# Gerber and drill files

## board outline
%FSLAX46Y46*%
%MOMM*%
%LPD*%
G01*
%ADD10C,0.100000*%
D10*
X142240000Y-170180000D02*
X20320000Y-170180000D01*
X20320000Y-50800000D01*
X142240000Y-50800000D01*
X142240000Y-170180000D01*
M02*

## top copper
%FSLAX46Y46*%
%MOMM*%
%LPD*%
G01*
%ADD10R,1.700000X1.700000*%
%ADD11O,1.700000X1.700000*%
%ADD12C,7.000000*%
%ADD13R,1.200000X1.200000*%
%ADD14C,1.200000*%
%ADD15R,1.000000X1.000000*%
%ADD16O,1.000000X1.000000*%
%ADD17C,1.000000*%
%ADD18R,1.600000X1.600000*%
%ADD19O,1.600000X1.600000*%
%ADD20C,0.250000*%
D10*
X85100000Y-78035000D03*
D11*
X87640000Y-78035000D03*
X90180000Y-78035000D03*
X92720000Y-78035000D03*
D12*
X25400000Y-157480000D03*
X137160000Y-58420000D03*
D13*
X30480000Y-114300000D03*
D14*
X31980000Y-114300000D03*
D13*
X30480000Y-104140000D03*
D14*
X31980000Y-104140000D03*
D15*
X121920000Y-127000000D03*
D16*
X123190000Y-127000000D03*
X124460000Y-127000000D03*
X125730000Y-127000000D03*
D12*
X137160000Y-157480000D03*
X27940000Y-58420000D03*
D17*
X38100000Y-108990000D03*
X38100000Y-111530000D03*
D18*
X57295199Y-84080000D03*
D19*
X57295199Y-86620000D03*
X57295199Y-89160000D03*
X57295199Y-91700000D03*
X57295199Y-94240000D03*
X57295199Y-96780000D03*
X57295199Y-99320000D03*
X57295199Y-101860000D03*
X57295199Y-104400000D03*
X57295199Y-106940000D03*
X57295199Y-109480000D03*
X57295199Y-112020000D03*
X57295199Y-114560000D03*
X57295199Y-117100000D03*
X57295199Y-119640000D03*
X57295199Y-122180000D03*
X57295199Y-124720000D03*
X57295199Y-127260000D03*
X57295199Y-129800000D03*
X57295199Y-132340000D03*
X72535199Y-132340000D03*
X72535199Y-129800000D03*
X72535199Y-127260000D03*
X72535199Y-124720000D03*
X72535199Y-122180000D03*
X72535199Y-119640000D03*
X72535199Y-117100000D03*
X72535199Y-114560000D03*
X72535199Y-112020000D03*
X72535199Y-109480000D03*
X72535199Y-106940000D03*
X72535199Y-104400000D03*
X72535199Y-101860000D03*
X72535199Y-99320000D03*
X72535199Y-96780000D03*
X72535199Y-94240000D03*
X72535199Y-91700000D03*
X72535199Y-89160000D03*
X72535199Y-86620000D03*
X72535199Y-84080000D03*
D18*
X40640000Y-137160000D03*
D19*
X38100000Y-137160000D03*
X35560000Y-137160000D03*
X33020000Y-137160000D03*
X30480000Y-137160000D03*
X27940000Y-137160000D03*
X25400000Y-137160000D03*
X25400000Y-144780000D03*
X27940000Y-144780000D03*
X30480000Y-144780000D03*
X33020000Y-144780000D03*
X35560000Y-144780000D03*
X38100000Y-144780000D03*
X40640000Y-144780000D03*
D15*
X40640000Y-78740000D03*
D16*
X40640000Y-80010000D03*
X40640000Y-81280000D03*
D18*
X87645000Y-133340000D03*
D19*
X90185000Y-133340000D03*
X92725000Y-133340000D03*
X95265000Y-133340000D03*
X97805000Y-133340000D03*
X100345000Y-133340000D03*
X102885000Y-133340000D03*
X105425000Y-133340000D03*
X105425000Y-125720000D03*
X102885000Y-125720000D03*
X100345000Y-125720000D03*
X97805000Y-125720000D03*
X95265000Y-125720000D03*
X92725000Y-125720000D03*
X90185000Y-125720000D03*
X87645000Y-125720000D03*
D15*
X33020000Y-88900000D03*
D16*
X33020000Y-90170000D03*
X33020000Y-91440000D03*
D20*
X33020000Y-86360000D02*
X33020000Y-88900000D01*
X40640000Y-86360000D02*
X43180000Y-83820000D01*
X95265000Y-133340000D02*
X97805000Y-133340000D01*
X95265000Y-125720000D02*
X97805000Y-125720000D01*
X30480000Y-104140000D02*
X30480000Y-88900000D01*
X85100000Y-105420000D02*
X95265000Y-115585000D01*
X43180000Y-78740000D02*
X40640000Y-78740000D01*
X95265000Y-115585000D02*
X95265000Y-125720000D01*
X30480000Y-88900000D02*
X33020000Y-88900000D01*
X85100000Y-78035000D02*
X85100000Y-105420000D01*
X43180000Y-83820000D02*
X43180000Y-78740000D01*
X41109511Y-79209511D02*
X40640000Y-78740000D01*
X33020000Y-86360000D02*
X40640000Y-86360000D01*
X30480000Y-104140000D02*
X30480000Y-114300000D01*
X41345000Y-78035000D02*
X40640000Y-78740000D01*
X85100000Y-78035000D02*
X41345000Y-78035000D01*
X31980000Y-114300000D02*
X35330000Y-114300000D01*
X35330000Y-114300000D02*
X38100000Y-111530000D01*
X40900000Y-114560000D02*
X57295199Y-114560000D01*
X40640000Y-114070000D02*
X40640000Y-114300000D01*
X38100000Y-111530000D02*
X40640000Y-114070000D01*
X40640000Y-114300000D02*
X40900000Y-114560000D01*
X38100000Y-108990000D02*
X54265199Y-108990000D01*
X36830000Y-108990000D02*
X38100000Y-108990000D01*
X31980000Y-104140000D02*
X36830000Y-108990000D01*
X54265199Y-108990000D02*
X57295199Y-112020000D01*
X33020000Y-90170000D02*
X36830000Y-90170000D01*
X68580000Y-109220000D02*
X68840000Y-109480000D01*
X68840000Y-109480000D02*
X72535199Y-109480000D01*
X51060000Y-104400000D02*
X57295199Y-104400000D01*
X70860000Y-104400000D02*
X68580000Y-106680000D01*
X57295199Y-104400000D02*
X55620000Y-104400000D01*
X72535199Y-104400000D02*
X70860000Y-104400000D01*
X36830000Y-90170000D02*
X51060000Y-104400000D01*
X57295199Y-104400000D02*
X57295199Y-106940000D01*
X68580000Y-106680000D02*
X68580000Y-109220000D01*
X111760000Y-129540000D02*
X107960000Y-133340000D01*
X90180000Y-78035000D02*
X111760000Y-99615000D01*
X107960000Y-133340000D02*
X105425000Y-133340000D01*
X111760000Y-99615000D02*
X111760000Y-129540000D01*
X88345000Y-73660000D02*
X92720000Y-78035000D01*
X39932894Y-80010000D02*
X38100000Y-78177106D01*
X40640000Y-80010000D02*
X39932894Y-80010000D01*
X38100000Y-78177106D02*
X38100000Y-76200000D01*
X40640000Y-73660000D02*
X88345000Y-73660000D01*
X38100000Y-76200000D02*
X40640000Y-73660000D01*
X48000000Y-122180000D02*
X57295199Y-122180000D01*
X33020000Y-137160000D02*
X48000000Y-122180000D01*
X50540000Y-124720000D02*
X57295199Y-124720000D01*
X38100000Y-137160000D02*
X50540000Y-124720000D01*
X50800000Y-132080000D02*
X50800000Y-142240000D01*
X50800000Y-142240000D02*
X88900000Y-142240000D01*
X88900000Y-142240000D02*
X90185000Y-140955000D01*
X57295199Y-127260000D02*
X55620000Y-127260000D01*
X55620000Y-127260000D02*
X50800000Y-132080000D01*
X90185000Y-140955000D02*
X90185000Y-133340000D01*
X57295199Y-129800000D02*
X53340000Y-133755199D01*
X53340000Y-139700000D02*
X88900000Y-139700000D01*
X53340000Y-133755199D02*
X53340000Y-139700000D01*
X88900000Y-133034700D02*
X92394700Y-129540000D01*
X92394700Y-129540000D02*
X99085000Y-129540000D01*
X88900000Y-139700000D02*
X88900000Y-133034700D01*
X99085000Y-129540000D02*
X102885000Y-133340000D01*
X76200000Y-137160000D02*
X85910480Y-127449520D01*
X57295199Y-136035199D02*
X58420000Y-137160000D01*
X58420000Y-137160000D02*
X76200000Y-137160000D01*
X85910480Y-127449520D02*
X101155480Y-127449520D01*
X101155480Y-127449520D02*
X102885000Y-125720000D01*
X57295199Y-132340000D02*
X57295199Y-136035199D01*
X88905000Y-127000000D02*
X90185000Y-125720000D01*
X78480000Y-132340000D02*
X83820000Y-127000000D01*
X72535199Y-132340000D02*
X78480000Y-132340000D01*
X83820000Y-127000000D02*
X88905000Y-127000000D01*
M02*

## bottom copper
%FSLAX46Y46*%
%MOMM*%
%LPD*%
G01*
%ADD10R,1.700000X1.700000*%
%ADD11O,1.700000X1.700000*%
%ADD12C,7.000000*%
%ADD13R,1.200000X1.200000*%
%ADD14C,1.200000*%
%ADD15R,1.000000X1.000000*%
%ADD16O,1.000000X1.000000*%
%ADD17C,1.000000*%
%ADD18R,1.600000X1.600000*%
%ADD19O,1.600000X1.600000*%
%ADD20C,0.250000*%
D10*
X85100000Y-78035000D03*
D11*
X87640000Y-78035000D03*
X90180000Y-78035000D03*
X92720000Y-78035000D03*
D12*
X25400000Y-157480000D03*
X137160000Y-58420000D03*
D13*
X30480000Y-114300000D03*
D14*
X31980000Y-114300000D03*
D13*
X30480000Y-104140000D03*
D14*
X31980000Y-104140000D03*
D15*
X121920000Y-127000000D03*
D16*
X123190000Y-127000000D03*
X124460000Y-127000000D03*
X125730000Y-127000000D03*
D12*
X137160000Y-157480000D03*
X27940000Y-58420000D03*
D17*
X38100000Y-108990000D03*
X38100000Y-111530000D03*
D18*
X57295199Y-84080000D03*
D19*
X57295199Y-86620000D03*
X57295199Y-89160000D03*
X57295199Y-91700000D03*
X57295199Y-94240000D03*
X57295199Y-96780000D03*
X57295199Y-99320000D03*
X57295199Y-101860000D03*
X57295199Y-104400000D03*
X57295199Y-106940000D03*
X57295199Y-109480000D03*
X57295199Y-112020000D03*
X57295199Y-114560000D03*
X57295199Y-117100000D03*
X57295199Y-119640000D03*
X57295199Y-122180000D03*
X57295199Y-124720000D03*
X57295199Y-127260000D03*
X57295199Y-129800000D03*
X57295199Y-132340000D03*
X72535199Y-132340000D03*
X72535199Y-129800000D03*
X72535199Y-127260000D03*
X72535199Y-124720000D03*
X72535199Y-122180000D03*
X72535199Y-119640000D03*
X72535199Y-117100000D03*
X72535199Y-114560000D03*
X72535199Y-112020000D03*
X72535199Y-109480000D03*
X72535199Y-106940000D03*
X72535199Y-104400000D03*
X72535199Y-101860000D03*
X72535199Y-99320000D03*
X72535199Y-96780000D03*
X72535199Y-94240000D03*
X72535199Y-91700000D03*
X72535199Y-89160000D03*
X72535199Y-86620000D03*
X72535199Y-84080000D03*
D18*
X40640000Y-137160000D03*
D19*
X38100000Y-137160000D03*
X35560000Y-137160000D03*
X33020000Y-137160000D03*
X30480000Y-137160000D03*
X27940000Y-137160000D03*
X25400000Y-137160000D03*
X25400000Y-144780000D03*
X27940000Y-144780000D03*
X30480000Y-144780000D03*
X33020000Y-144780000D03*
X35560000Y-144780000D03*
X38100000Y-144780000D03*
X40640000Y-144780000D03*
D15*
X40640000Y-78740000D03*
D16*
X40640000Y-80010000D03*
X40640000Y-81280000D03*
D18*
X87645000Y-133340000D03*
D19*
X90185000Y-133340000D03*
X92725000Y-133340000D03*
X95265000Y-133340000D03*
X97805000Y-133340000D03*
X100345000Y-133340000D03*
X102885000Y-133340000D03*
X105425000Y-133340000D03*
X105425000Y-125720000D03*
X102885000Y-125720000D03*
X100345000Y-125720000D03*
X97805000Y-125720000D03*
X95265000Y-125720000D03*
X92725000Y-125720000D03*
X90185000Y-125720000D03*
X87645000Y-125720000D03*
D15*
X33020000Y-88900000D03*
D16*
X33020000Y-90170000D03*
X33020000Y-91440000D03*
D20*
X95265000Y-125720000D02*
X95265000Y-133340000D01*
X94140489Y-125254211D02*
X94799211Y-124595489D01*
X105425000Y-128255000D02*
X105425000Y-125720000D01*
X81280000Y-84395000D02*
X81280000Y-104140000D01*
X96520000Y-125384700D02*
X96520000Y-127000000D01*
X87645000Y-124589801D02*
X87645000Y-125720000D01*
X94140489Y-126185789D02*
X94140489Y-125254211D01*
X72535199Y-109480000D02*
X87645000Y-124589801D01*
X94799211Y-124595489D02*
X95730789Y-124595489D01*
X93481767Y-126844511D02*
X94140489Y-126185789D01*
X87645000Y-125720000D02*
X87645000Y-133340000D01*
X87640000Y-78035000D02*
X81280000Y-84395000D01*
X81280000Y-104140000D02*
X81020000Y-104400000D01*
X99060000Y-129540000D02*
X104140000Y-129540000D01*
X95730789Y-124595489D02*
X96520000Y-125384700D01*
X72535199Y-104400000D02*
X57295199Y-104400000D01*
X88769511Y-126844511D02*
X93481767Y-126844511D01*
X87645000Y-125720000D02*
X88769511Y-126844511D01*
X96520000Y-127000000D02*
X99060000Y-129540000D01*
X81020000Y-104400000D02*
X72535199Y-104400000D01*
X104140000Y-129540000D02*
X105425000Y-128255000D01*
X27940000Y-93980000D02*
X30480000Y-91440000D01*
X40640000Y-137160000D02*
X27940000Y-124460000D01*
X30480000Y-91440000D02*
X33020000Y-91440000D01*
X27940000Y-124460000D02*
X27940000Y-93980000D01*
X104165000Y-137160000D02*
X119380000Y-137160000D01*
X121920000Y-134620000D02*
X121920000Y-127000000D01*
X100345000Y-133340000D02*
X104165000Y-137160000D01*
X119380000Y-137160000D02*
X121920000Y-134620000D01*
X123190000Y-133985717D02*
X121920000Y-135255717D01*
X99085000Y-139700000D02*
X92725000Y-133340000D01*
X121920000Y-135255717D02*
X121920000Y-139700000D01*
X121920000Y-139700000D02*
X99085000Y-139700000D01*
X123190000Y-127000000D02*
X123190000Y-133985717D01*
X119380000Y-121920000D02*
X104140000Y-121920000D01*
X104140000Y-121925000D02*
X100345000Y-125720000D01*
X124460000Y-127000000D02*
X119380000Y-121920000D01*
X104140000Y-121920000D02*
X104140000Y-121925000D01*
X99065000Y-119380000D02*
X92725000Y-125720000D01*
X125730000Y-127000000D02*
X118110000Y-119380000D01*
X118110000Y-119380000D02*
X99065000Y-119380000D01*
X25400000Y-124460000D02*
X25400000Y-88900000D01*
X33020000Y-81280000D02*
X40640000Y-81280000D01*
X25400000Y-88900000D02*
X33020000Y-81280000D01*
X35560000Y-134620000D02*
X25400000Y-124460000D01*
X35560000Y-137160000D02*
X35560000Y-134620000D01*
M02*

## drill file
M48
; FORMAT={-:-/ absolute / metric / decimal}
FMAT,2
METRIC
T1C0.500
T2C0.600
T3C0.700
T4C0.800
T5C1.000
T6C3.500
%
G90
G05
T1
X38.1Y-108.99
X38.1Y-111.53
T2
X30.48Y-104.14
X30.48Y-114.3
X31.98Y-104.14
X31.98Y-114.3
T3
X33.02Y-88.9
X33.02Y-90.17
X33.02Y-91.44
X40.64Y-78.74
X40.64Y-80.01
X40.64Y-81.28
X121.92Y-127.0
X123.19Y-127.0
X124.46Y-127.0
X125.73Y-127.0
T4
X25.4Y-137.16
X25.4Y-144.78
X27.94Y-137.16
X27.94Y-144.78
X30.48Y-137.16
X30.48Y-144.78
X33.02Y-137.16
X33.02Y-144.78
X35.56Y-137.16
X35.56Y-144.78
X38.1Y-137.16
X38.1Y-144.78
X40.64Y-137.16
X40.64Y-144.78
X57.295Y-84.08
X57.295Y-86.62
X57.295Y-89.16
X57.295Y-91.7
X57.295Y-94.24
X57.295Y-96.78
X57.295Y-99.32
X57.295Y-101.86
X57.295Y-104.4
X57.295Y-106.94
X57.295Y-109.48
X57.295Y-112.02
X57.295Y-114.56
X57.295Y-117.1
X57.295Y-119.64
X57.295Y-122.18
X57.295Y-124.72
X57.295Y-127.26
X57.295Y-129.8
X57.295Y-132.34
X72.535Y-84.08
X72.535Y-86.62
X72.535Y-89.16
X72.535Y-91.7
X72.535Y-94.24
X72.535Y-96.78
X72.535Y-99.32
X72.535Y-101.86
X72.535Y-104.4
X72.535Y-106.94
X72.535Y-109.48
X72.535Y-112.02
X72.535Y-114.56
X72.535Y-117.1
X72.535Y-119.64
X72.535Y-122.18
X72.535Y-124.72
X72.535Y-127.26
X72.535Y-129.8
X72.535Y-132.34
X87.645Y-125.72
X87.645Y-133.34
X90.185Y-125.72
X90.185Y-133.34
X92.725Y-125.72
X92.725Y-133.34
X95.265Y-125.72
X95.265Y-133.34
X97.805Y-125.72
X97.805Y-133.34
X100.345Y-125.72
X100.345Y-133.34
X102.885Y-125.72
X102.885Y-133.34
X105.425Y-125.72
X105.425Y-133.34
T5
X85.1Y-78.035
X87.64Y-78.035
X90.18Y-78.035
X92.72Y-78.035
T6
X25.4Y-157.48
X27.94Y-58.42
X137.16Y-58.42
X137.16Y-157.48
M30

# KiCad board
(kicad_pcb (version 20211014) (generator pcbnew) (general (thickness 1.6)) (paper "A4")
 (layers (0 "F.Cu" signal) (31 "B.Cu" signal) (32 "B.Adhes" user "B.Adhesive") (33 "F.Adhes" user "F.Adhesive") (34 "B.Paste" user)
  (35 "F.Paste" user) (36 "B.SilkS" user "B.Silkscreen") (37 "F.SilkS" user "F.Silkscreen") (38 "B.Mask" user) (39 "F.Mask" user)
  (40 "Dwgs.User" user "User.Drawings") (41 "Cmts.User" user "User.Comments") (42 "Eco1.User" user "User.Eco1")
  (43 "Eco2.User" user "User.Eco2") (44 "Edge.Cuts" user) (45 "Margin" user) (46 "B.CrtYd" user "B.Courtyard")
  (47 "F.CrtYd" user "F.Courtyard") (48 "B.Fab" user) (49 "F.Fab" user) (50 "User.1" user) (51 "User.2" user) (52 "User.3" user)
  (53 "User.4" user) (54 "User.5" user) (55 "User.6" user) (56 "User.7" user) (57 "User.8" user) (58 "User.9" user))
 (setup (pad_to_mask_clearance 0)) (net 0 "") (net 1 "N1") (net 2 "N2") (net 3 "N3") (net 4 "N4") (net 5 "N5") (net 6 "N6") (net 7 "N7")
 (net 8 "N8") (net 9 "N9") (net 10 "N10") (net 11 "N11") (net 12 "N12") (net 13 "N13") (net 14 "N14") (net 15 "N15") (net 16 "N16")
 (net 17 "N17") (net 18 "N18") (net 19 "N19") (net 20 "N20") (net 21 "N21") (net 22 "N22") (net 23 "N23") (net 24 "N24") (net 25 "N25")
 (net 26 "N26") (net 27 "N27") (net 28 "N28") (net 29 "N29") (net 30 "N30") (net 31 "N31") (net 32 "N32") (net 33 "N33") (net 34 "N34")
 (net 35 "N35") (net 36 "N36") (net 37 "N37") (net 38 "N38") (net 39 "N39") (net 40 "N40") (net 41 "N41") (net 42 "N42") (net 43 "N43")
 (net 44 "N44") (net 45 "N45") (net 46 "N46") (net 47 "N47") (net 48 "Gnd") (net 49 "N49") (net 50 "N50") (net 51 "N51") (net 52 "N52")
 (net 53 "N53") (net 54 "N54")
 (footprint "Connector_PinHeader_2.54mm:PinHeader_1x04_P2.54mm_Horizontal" (layer "F.Cu") (at 85.1 78.035 90)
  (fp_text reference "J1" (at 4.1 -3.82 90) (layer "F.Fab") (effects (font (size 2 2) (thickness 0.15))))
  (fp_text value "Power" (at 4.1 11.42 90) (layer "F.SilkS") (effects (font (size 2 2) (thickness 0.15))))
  (pad "1" thru_hole rect (at 0 0 90) (size 1.7 1.7) (drill 1) (layers *.Cu *.Mask) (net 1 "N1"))
  (pad "2" thru_hole oval (at 0 2.54 90) (size 1.7 1.7) (drill 1) (layers *.Cu *.Mask) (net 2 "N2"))
  (pad "3" thru_hole oval (at 0 5.08 90) (size 1.7 1.7) (drill 1) (layers *.Cu *.Mask) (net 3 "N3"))
  (pad "4" thru_hole oval (at 0 7.62 90) (size 1.7 1.7) (drill 1) (layers *.Cu *.Mask) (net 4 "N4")))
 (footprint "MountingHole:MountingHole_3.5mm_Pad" (layer "F.Cu") (at 25.4 157.48)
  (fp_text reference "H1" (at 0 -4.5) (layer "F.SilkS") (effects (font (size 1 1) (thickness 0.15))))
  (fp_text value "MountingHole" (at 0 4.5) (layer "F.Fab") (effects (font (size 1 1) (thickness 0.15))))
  (pad "1" thru_hole circle (at 0 0) (size 7 7) (drill 3.5) (layers *.Cu *.Mask)))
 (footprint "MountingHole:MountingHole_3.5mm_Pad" (layer "F.Cu") (at 137.16 58.42)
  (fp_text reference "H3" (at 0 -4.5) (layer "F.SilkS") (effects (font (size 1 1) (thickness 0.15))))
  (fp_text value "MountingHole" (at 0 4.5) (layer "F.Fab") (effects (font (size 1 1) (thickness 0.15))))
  (pad "1" thru_hole circle (at 0 0) (size 7 7) (drill 3.5) (layers *.Cu *.Mask)))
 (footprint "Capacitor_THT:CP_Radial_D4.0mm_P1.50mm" (layer "F.Cu") (at 30.48 114.3)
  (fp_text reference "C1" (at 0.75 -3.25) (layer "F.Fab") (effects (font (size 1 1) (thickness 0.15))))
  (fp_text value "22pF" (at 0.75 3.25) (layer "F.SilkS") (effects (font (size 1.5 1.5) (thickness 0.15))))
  (pad "1" thru_hole rect (at 0 0) (size 1.2 1.2) (drill 0.6) (layers *.Cu *.Mask) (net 1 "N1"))
  (pad "2" thru_hole circle (at 1.5 0) (size 1.2 1.2) (drill 0.6) (layers *.Cu *.Mask) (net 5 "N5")))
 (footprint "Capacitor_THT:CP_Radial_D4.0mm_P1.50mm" (layer "F.Cu") (at 30.48 104.14)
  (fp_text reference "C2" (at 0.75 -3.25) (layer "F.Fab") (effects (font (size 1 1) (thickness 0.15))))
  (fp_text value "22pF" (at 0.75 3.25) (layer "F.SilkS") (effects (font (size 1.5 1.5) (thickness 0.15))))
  (pad "1" thru_hole rect (at 0 0) (size 1.2 1.2) (drill 0.6) (layers *.Cu *.Mask) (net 1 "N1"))
  (pad "2" thru_hole circle (at 1.5 0) (size 1.2 1.2) (drill 0.6) (layers *.Cu *.Mask) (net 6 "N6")))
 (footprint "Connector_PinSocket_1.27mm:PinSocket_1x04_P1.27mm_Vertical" (layer "F.Cu") (at 121.92 127 90)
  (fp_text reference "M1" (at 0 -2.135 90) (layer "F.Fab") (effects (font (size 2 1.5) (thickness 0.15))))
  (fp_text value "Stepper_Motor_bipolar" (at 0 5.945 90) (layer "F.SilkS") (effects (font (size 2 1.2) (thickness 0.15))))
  (pad "1" thru_hole rect (at 0 0 90) (size 1 1) (drill 0.7) (layers *.Cu *.Mask) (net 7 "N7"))
  (pad "2" thru_hole oval (at 0 1.27 90) (size 1 1) (drill 0.7) (layers *.Cu *.Mask) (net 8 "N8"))
  (pad "3" thru_hole oval (at 0 2.54 90) (size 1 1) (drill 0.7) (layers *.Cu *.Mask) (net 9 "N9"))
  (pad "4" thru_hole oval (at 0 3.81 90) (size 1 1) (drill 0.7) (layers *.Cu *.Mask) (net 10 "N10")))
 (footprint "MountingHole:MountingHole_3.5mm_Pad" (layer "F.Cu") (at 137.16 157.48)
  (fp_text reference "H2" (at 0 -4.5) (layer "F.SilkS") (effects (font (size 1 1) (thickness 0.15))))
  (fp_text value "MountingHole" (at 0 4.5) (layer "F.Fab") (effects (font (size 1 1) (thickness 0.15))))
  (pad "1" thru_hole circle (at 0 0) (size 7 7) (drill 3.5) (layers *.Cu *.Mask)))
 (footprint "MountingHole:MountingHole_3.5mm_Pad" (layer "F.Cu") (at 27.94 58.42)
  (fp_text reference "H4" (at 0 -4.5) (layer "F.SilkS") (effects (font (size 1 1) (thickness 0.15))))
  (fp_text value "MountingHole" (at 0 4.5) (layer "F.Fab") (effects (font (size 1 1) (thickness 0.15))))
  (pad "1" thru_hole circle (at 0 0) (size 7 7) (drill 3.5) (layers *.Cu *.Mask)))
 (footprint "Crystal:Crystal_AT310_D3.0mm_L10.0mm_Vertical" (layer "F.Cu") (at 38.1 108.99 -90)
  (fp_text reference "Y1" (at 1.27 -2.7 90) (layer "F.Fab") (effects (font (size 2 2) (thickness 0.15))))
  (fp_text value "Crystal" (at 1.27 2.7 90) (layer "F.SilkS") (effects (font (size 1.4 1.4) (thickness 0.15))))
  (pad "1" thru_hole circle (at 0 0 270) (size 1 1) (drill 0.5) (layers *.Cu *.Mask) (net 6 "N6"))
  (pad "2" thru_hole circle (at 2.54 0 270) (size 1 1) (drill 0.5) (layers *.Cu *.Mask) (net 5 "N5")))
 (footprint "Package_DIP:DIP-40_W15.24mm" (layer "F.Cu") (at 57.295199 84.08)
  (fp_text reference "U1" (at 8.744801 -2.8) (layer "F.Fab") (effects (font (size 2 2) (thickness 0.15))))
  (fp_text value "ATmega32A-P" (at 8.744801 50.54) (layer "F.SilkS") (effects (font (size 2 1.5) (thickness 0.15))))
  (pad "1" thru_hole rect (at 0 0) (size 1.6 1.6) (drill 0.8) (layers *.Cu *.Mask) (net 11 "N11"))
  (pad "2" thru_hole oval (at 0 2.54) (size 1.6 1.6) (drill 0.8) (layers *.Cu *.Mask) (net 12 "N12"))
  (pad "3" thru_hole oval (at 0 5.08) (size 1.6 1.6) (drill 0.8) (layers *.Cu *.Mask) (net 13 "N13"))
  (pad "4" thru_hole oval (at 0 7.62) (size 1.6 1.6) (drill 0.8) (layers *.Cu *.Mask) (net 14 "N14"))
  (pad "5" thru_hole oval (at 0 10.16) (size 1.6 1.6) (drill 0.8) (layers *.Cu *.Mask) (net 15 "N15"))
  (pad "6" thru_hole oval (at 0 12.7) (size 1.6 1.6) (drill 0.8) (layers *.Cu *.Mask) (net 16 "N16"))
  (pad "7" thru_hole oval (at 0 15.24) (size 1.6 1.6) (drill 0.8) (layers *.Cu *.Mask) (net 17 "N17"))
  (pad "8" thru_hole oval (at 0 17.78) (size 1.6 1.6) (drill 0.8) (layers *.Cu *.Mask) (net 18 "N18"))
  (pad "9" thru_hole oval (at 0 20.32) (size 1.6 1.6) (drill 0.8) (layers *.Cu *.Mask) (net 2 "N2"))
  (pad "10" thru_hole oval (at 0 22.86) (size 1.6 1.6) (drill 0.8) (layers *.Cu *.Mask) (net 2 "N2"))
  (pad "11" thru_hole oval (at 0 25.4) (size 1.6 1.6) (drill 0.8) (layers *.Cu *.Mask) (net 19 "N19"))
  (pad "12" thru_hole oval (at 0 27.94) (size 1.6 1.6) (drill 0.8) (layers *.Cu *.Mask) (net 6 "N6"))
  (pad "13" thru_hole oval (at 0 30.48) (size 1.6 1.6) (drill 0.8) (layers *.Cu *.Mask) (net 5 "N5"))
  (pad "14" thru_hole oval (at 0 33.02) (size 1.6 1.6) (drill 0.8) (layers *.Cu *.Mask) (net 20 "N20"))
  (pad "15" thru_hole oval (at 0 35.56) (size 1.6 1.6) (drill 0.8) (layers *.Cu *.Mask) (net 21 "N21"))
  (pad "16" thru_hole oval (at 0 38.1) (size 1.6 1.6) (drill 0.8) (layers *.Cu *.Mask) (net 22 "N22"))
  (pad "17" thru_hole oval (at 0 40.64) (size 1.6 1.6) (drill 0.8) (layers *.Cu *.Mask) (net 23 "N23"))
  (pad "18" thru_hole oval (at 0 43.18) (size 1.6 1.6) (drill 0.8) (layers *.Cu *.Mask) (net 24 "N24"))
  (pad "19" thru_hole oval (at 0 45.72) (size 1.6 1.6) (drill 0.8) (layers *.Cu *.Mask) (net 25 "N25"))
  (pad "20" thru_hole oval (at 0 48.26) (size 1.6 1.6) (drill 0.8) (layers *.Cu *.Mask) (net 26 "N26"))
  (pad "21" thru_hole oval (at 15.24 48.26) (size 1.6 1.6) (drill 0.8) (layers *.Cu *.Mask) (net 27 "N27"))
  (pad "22" thru_hole oval (at 15.24 45.72) (size 1.6 1.6) (drill 0.8) (layers *.Cu *.Mask) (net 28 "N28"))
  (pad "23" thru_hole oval (at 15.24 43.18) (size 1.6 1.6) (drill 0.8) (layers *.Cu *.Mask) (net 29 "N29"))
  (pad "24" thru_hole oval (at 15.24 40.64) (size 1.6 1.6) (drill 0.8) (layers *.Cu *.Mask) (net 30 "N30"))
  (pad "25" thru_hole oval (at 15.24 38.1) (size 1.6 1.6) (drill 0.8) (layers *.Cu *.Mask) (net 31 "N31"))
  (pad "26" thru_hole oval (at 15.24 35.56) (size 1.6 1.6) (drill 0.8) (layers *.Cu *.Mask) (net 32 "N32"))
  (pad "27" thru_hole oval (at 15.24 33.02) (size 1.6 1.6) (drill 0.8) (layers *.Cu *.Mask) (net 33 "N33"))
  (pad "28" thru_hole oval (at 15.24 30.48) (size 1.6 1.6) (drill 0.8) (layers *.Cu *.Mask) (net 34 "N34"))
  (pad "29" thru_hole oval (at 15.24 27.94) (size 1.6 1.6) (drill 0.8) (layers *.Cu *.Mask) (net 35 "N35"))
  (pad "30" thru_hole oval (at 15.24 25.4) (size 1.6 1.6) (drill 0.8) (layers *.Cu *.Mask) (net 2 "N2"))
  (pad "31" thru_hole oval (at 15.24 22.86) (size 1.6 1.6) (drill 0.8) (layers *.Cu *.Mask) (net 19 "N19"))
  (pad "32" thru_hole oval (at 15.24 20.32) (size 1.6 1.6) (drill 0.8) (layers *.Cu *.Mask) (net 2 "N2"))
  (pad "33" thru_hole oval (at 15.24 17.78) (size 1.6 1.6) (drill 0.8) (layers *.Cu *.Mask) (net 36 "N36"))
  (pad "34" thru_hole oval (at 15.24 15.24) (size 1.6 1.6) (drill 0.8) (layers *.Cu *.Mask) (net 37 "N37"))
  (pad "35" thru_hole oval (at 15.24 12.7) (size 1.6 1.6) (drill 0.8) (layers *.Cu *.Mask) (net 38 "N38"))
  (pad "36" thru_hole oval (at 15.24 10.16) (size 1.6 1.6) (drill 0.8) (layers *.Cu *.Mask) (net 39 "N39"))
  (pad "37" thru_hole oval (at 15.24 7.62) (size 1.6 1.6) (drill 0.8) (layers *.Cu *.Mask) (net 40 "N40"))
  (pad "38" thru_hole oval (at 15.24 5.08) (size 1.6 1.6) (drill 0.8) (layers *.Cu *.Mask) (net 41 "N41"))
  (pad "39" thru_hole oval (at 15.24 2.54) (size 1.6 1.6) (drill 0.8) (layers *.Cu *.Mask) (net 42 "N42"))
  (pad "40" thru_hole oval (at 15.24 0) (size 1.6 1.6) (drill 0.8) (layers *.Cu *.Mask) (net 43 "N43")))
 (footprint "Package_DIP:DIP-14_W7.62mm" (layer "F.Cu") (at 40.64 137.16 -90)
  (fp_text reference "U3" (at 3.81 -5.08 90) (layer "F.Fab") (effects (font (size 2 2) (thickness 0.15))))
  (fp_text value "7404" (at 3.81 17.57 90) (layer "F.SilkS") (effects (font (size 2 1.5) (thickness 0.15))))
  (pad "1" thru_hole rect (at 0 0 270) (size 1.6 1.6) (drill 0.8) (layers *.Cu *.Mask) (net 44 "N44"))
  (pad "2" thru_hole oval (at 0 2.54 270) (size 1.6 1.6) (drill 0.8) (layers *.Cu *.Mask) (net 23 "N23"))
  (pad "3" thru_hole oval (at 0 5.08 270) (size 1.6 1.6) (drill 0.8) (layers *.Cu *.Mask) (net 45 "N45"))
  (pad "4" thru_hole oval (at 0 7.62 270) (size 1.6 1.6) (drill 0.8) (layers *.Cu *.Mask) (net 22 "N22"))
  (pad "5" thru_hole oval (at 0 10.16 270) (size 1.6 1.6) (drill 0.8) (layers *.Cu *.Mask) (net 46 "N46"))
  (pad "6" thru_hole oval (at 0 12.7 270) (size 1.6 1.6) (drill 0.8) (layers *.Cu *.Mask) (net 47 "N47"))
  (pad "7" thru_hole oval (at 0 15.24 270) (size 1.6 1.6) (drill 0.8) (layers *.Cu *.Mask) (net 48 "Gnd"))
  (pad "8" thru_hole oval (at 7.62 15.24 270) (size 1.6 1.6) (drill 0.8) (layers *.Cu *.Mask) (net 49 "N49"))
  (pad "9" thru_hole oval (at 7.62 12.7 270) (size 1.6 1.6) (drill 0.8) (layers *.Cu *.Mask) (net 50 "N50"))
  (pad "10" thru_hole oval (at 7.62 10.16 270) (size 1.6 1.6) (drill 0.8) (layers *.Cu *.Mask) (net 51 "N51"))
  (pad "11" thru_hole oval (at 7.62 7.62 270) (size 1.6 1.6) (drill 0.8) (layers *.Cu *.Mask) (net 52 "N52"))
  (pad "12" thru_hole oval (at 7.62 5.08 270) (size 1.6 1.6) (drill 0.8) (layers *.Cu *.Mask) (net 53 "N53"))
  (pad "13" thru_hole oval (at 7.62 2.54 270) (size 1.6 1.6) (drill 0.8) (layers *.Cu *.Mask) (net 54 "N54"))
  (pad "14" thru_hole oval (at 7.62 0 270) (size 1.6 1.6) (drill 0.8) (layers *.Cu *.Mask) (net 48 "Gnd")))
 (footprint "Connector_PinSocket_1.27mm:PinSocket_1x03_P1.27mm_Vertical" (layer "F.Cu") (at 40.64 78.74)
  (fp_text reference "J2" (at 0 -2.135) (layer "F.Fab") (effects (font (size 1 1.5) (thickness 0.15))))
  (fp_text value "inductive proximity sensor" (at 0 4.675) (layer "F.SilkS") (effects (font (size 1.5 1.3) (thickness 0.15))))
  (pad "1" thru_hole rect (at 0 0) (size 1 1) (drill 0.7) (layers *.Cu *.Mask) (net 1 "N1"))
  (pad "2" thru_hole oval (at 0 1.27) (size 1 1) (drill 0.7) (layers *.Cu *.Mask) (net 4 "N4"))
  (pad "3" thru_hole oval (at 0 2.54) (size 1 1) (drill 0.7) (layers *.Cu *.Mask) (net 45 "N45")))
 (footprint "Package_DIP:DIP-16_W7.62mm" (layer "F.Cu") (at 87.645 133.34 90)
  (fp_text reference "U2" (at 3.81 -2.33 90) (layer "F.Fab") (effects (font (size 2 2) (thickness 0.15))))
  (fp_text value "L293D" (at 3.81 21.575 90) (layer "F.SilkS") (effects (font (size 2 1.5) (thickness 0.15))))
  (pad "1" thru_hole rect (at 0 0 90) (size 1.6 1.6) (drill 0.8) (layers *.Cu *.Mask) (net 2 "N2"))
  (pad "2" thru_hole oval (at 0 2.54 90) (size 1.6 1.6) (drill 0.8) (layers *.Cu *.Mask) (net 24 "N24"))
  (pad "3" thru_hole oval (at 0 5.08 90) (size 1.6 1.6) (drill 0.8) (layers *.Cu *.Mask) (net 8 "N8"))
  (pad "4" thru_hole oval (at 0 7.62 90) (size 1.6 1.6) (drill 0.8) (layers *.Cu *.Mask) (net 1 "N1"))
  (pad "5" thru_hole oval (at 0 10.16 90) (size 1.6 1.6) (drill 0.8) (layers *.Cu *.Mask) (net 1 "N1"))
  (pad "6" thru_hole oval (at 0 12.7 90) (size 1.6 1.6) (drill 0.8) (layers *.Cu *.Mask) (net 7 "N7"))
  (pad "7" thru_hole oval (at 0 15.24 90) (size 1.6 1.6) (drill 0.8) (layers *.Cu *.Mask) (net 25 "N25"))
  (pad "8" thru_hole oval (at 0 17.78 90) (size 1.6 1.6) (drill 0.8) (layers *.Cu *.Mask) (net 3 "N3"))
  (pad "9" thru_hole oval (at 7.62 17.78 90) (size 1.6 1.6) (drill 0.8) (layers *.Cu *.Mask) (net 2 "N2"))
  (pad "10" thru_hole oval (at 7.62 15.24 90) (size 1.6 1.6) (drill 0.8) (layers *.Cu *.Mask) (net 26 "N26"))
  (pad "11" thru_hole oval (at 7.62 12.7 90) (size 1.6 1.6) (drill 0.8) (layers *.Cu *.Mask) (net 9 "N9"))
  (pad "12" thru_hole oval (at 7.62 10.16 90) (size 1.6 1.6) (drill 0.8) (layers *.Cu *.Mask) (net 1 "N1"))
  (pad "13" thru_hole oval (at 7.62 7.62 90) (size 1.6 1.6) (drill 0.8) (layers *.Cu *.Mask) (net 1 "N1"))
  (pad "14" thru_hole oval (at 7.62 5.08 90) (size 1.6 1.6) (drill 0.8) (layers *.Cu *.Mask) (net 10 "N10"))
  (pad "15" thru_hole oval (at 7.62 2.54 90) (size 1.6 1.6) (drill 0.8) (layers *.Cu *.Mask) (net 27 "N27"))
  (pad "16" thru_hole oval (at 7.62 0 90) (size 1.6 1.6) (drill 0.8) (layers *.Cu *.Mask) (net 2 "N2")))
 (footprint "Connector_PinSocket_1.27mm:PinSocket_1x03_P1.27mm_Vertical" (layer "F.Cu") (at 33.02 88.9)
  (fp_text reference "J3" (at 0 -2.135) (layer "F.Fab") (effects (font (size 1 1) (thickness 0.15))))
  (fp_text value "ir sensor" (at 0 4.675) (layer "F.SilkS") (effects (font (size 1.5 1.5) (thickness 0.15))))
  (pad "1" thru_hole rect (at 0 0) (size 1 1) (drill 0.7) (layers *.Cu *.Mask) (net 1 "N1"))
  (pad "2" thru_hole oval (at 0 1.27) (size 1 1) (drill 0.7) (layers *.Cu *.Mask) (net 2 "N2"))
  (pad "3" thru_hole oval (at 0 2.54) (size 1 1) (drill 0.7) (layers *.Cu *.Mask) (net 44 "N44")))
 (gr_poly (pts (xy 142.24 170.18) (xy 20.32 170.18) (xy 20.32 50.8) (xy 142.24 50.8)) (layer "Edge.Cuts") (width 0.1) (fill none))
 (segment (start 33.02 86.36) (end 33.02 88.9) (width 0.25) (layer "F.Cu") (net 1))
 (segment (start 40.64 86.36) (end 43.18 83.82) (width 0.25) (layer "F.Cu") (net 1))
 (segment (start 95.265 133.34) (end 97.805 133.34) (width 0.25) (layer "F.Cu") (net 1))
 (segment (start 95.265 125.72) (end 97.805 125.72) (width 0.25) (layer "F.Cu") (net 1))
 (segment (start 30.48 104.14) (end 30.48 88.9) (width 0.25) (layer "F.Cu") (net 1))
 (segment (start 85.1 105.42) (end 95.265 115.585) (width 0.25) (layer "F.Cu") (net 1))
 (segment (start 43.18 78.74) (end 40.64 78.74) (width 0.25) (layer "F.Cu") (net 1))
 (segment (start 95.265 115.585) (end 95.265 125.72) (width 0.25) (layer "F.Cu") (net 1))
 (segment (start 30.48 88.9) (end 33.02 88.9) (width 0.25) (layer "F.Cu") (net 1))
 (segment (start 85.1 78.035) (end 85.1 105.42) (width 0.25) (layer "F.Cu") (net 1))
 (segment (start 43.18 83.82) (end 43.18 78.74) (width 0.25) (layer "F.Cu") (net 1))
 (segment (start 41.109511 79.209511) (end 40.64 78.74) (width 0.25) (layer "F.Cu") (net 1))
 (segment (start 33.02 86.36) (end 40.64 86.36) (width 0.25) (layer "F.Cu") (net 1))
 (segment (start 30.48 104.14) (end 30.48 114.3) (width 0.25) (layer "F.Cu") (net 1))
 (segment (start 41.345 78.035) (end 40.64 78.74) (width 0.25) (layer "F.Cu") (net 1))
 (segment (start 85.1 78.035) (end 41.345 78.035) (width 0.25) (layer "F.Cu") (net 1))
 (segment (start 95.265 125.72) (end 95.265 133.34) (width 0.25) (layer "B.Cu") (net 1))
 (segment (start 31.98 114.3) (end 35.33 114.3) (width 0.25) (layer "F.Cu") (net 5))
 (segment (start 35.33 114.3) (end 38.1 111.53) (width 0.25) (layer "F.Cu") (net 5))
 (segment (start 40.9 114.56) (end 57.295199 114.56) (width 0.25) (layer "F.Cu") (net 5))
 (segment (start 40.64 114.07) (end 40.64 114.3) (width 0.25) (layer "F.Cu") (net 5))
 (segment (start 38.1 111.53) (end 40.64 114.07) (width 0.25) (layer "F.Cu") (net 5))
 (segment (start 40.64 114.3) (end 40.9 114.56) (width 0.25) (layer "F.Cu") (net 5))
 (segment (start 38.1 108.99) (end 54.265199 108.99) (width 0.25) (layer "F.Cu") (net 6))
 (segment (start 36.83 108.99) (end 38.1 108.99) (width 0.25) (layer "F.Cu") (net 6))
 (segment (start 31.98 104.14) (end 36.83 108.99) (width 0.25) (layer "F.Cu") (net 6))
 (segment (start 54.265199 108.99) (end 57.295199 112.02) (width 0.25) (layer "F.Cu") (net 6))
 (segment (start 33.02 90.17) (end 36.83 90.17) (width 0.25) (layer "F.Cu") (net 2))
 (segment (start 68.58 109.22) (end 68.84 109.48) (width 0.25) (layer "F.Cu") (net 2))
 (segment (start 68.84 109.48) (end 72.535199 109.48) (width 0.25) (layer "F.Cu") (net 2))
 (segment (start 51.06 104.4) (end 57.295199 104.4) (width 0.25) (layer "F.Cu") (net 2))
 (segment (start 70.86 104.4) (end 68.58 106.68) (width 0.25) (layer "F.Cu") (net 2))
 (segment (start 57.295199 104.4) (end 55.62 104.4) (width 0.25) (layer "F.Cu") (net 2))
 (segment (start 72.535199 104.4) (end 70.86 104.4) (width 0.25) (layer "F.Cu") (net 2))
 (segment (start 36.83 90.17) (end 51.06 104.4) (width 0.25) (layer "F.Cu") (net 2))
 (segment (start 57.295199 104.4) (end 57.295199 106.94) (width 0.25) (layer "F.Cu") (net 2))
 (segment (start 68.58 106.68) (end 68.58 109.22) (width 0.25) (layer "F.Cu") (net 2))
 (segment (start 94.140489 125.254211) (end 94.799211 124.595489) (width 0.25) (layer "B.Cu") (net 2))
 (segment (start 105.425 128.255) (end 105.425 125.72) (width 0.25) (layer "B.Cu") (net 2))
 (segment (start 81.28 84.395) (end 81.28 104.14) (width 0.25) (layer "B.Cu") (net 2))
 (segment (start 96.52 125.3847) (end 96.52 127) (width 0.25) (layer "B.Cu") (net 2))
 (segment (start 87.645 124.589801) (end 87.645 125.72) (width 0.25) (layer "B.Cu") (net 2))
 (segment (start 94.140489 126.185789) (end 94.140489 125.254211) (width 0.25) (layer "B.Cu") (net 2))
 (segment (start 72.535199 109.48) (end 87.645 124.589801) (width 0.25) (layer "B.Cu") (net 2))
 (segment (start 94.799211 124.595489) (end 95.730789 124.595489) (width 0.25) (layer "B.Cu") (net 2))
 (segment (start 93.481767 126.844511) (end 94.140489 126.185789) (width 0.25) (layer "B.Cu") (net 2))
 (segment (start 87.645 125.72) (end 87.645 133.34) (width 0.25) (layer "B.Cu") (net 2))
 (segment (start 87.64 78.035) (end 81.28 84.395) (width 0.25) (layer "B.Cu") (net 2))
 (segment (start 81.28 104.14) (end 81.02 104.4) (width 0.25) (layer "B.Cu") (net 2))
 (segment (start 99.06 129.54) (end 104.14 129.54) (width 0.25) (layer "B.Cu") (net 2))
 (segment (start 95.730789 124.595489) (end 96.52 125.3847) (width 0.25) (layer "B.Cu") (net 2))
 (segment (start 72.535199 104.4) (end 57.295199 104.4) (width 0.25) (layer "B.Cu") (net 2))
 (segment (start 88.769511 126.844511) (end 93.481767 126.844511) (width 0.25) (layer "B.Cu") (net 2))
 (segment (start 87.645 125.72) (end 88.769511 126.844511) (width 0.25) (layer "B.Cu") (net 2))
 (segment (start 96.52 127) (end 99.06 129.54) (width 0.25) (layer "B.Cu") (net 2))
 (segment (start 81.02 104.4) (end 72.535199 104.4) (width 0.25) (layer "B.Cu") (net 2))
 (segment (start 104.14 129.54) (end 105.425 128.255) (width 0.25) (layer "B.Cu") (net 2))
 (segment (start 111.76 129.54) (end 107.96 133.34) (width 0.25) (layer "F.Cu") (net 3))
 (segment (start 90.18 78.035) (end 111.76 99.615) (width 0.25) (layer "F.Cu") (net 3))
 (segment (start 107.96 133.34) (end 105.425 133.34) (width 0.25) (layer "F.Cu") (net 3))
 (segment (start 111.76 99.615) (end 111.76 129.54) (width 0.25) (layer "F.Cu") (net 3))
 (segment (start 88.345 73.66) (end 92.72 78.035) (width 0.25) (layer "F.Cu") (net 4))
 (segment (start 39.932894 80.01) (end 38.1 78.177106) (width 0.25) (layer "F.Cu") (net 4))
 (segment (start 40.64 80.01) (end 39.932894 80.01) (width 0.25) (layer "F.Cu") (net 4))
 (segment (start 38.1 78.177106) (end 38.1 76.2) (width 0.25) (layer "F.Cu") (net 4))
 (segment (start 40.64 73.66) (end 88.345 73.66) (width 0.25) (layer "F.Cu") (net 4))
 (segment (start 38.1 76.2) (end 40.64 73.66) (width 0.25) (layer "F.Cu") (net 4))
 (segment (start 27.94 93.98) (end 30.48 91.44) (width 0.25) (layer "B.Cu") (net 44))
 (segment (start 40.64 137.16) (end 27.94 124.46) (width 0.25) (layer "B.Cu") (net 44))
 (segment (start 30.48 91.44) (end 33.02 91.44) (width 0.25) (layer "B.Cu") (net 44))
 (segment (start 27.94 124.46) (end 27.94 93.98) (width 0.25) (layer "B.Cu") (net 44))
 (segment (start 104.165 137.16) (end 119.38 137.16) (width 0.25) (layer "B.Cu") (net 7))
 (segment (start 121.92 134.62) (end 121.92 127) (width 0.25) (layer "B.Cu") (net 7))
 (segment (start 100.345 133.34) (end 104.165 137.16) (width 0.25) (layer "B.Cu") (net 7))
 (segment (start 119.38 137.16) (end 121.92 134.62) (width 0.25) (layer "B.Cu") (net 7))
 (segment (start 123.19 133.985717) (end 121.92 135.255717) (width 0.25) (layer "B.Cu") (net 8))
 (segment (start 99.085 139.7) (end 92.725 133.34) (width 0.25) (layer "B.Cu") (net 8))
 (segment (start 121.92 135.255717) (end 121.92 139.7) (width 0.25) (layer "B.Cu") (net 8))
 (segment (start 121.92 139.7) (end 99.085 139.7) (width 0.25) (layer "B.Cu") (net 8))
 (segment (start 123.19 127) (end 123.19 133.985717) (width 0.25) (layer "B.Cu") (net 8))
 (segment (start 119.38 121.92) (end 104.14 121.92) (width 0.25) (layer "B.Cu") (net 9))
 (segment (start 104.14 121.925) (end 100.345 125.72) (width 0.25) (layer "B.Cu") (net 9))
 (segment (start 124.46 127) (end 119.38 121.92) (width 0.25) (layer "B.Cu") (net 9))
 (segment (start 104.14 121.92) (end 104.14 121.925) (width 0.25) (layer "B.Cu") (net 9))
 (segment (start 99.065 119.38) (end 92.725 125.72) (width 0.25) (layer "B.Cu") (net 10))
 (segment (start 125.73 127) (end 118.11 119.38) (width 0.25) (layer "B.Cu") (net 10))
 (segment (start 118.11 119.38) (end 99.065 119.38) (width 0.25) (layer "B.Cu") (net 10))
 (segment (start 48 122.18) (end 57.295199 122.18) (width 0.25) (layer "F.Cu") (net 22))
 (segment (start 33.02 137.16) (end 48 122.18) (width 0.25) (layer "F.Cu") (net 22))
 (segment (start 50.54 124.72) (end 57.295199 124.72) (width 0.25) (layer "F.Cu") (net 23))
 (segment (start 38.1 137.16) (end 50.54 124.72) (width 0.25) (layer "F.Cu") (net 23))
 (segment (start 50.8 132.08) (end 50.8 142.24) (width 0.25) (layer "F.Cu") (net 24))
 (segment (start 50.8 142.24) (end 88.9 142.24) (width 0.25) (layer "F.Cu") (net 24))
 (segment (start 88.9 142.24) (end 90.185 140.955) (width 0.25) (layer "F.Cu") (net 24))
 (segment (start 57.295199 127.26) (end 55.62 127.26) (width 0.25) (layer "F.Cu") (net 24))
 (segment (start 55.62 127.26) (end 50.8 132.08) (width 0.25) (layer "F.Cu") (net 24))
 (segment (start 90.185 140.955) (end 90.185 133.34) (width 0.25) (layer "F.Cu") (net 24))
 (segment (start 57.295199 129.8) (end 53.34 133.755199) (width 0.25) (layer "F.Cu") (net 25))
 (segment (start 53.34 139.7) (end 88.9 139.7) (width 0.25) (layer "F.Cu") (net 25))
 (segment (start 53.34 133.755199) (end 53.34 139.7) (width 0.25) (layer "F.Cu") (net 25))
 (segment (start 88.9 133.0347) (end 92.3947 129.54) (width 0.25) (layer "F.Cu") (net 25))
 (segment (start 92.3947 129.54) (end 99.085 129.54) (width 0.25) (layer "F.Cu") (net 25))
 (segment (start 88.9 139.7) (end 88.9 133.0347) (width 0.25) (layer "F.Cu") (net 25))
 (segment (start 99.085 129.54) (end 102.885 133.34) (width 0.25) (layer "F.Cu") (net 25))
 (segment (start 76.2 137.16) (end 85.91048 127.44952) (width 0.25) (layer "F.Cu") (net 26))
 (segment (start 57.295199 136.035199) (end 58.42 137.16) (width 0.25) (layer "F.Cu") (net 26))
 (segment (start 58.42 137.16) (end 76.2 137.16) (width 0.25) (layer "F.Cu") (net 26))
 (segment (start 85.91048 127.44952) (end 101.15548 127.44952) (width 0.25) (layer "F.Cu") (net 26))
 (segment (start 101.15548 127.44952) (end 102.885 125.72) (width 0.25) (layer "F.Cu") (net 26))
 (segment (start 57.295199 132.34) (end 57.295199 136.035199) (width 0.25) (layer "F.Cu") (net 26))
 (segment (start 88.905 127) (end 90.185 125.72) (width 0.25) (layer "F.Cu") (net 27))
 (segment (start 78.48 132.34) (end 83.82 127) (width 0.25) (layer "F.Cu") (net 27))
 (segment (start 72.535199 132.34) (end 78.48 132.34) (width 0.25) (layer "F.Cu") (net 27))
 (segment (start 83.82 127) (end 88.905 127) (width 0.25) (layer "F.Cu") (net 27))
 (segment (start 25.4 124.46) (end 25.4 88.9) (width 0.25) (layer "B.Cu") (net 45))
 (segment (start 33.02 81.28) (end 40.64 81.28) (width 0.25) (layer "B.Cu") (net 45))
 (segment (start 25.4 88.9) (end 33.02 81.28) (width 0.25) (layer "B.Cu") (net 45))
 (segment (start 35.56 134.62) (end 25.4 124.46) (width 0.25) (layer "B.Cu") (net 45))
 (segment (start 35.56 137.16) (end 35.56 134.62) (width 0.25) (layer "B.Cu") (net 45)))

